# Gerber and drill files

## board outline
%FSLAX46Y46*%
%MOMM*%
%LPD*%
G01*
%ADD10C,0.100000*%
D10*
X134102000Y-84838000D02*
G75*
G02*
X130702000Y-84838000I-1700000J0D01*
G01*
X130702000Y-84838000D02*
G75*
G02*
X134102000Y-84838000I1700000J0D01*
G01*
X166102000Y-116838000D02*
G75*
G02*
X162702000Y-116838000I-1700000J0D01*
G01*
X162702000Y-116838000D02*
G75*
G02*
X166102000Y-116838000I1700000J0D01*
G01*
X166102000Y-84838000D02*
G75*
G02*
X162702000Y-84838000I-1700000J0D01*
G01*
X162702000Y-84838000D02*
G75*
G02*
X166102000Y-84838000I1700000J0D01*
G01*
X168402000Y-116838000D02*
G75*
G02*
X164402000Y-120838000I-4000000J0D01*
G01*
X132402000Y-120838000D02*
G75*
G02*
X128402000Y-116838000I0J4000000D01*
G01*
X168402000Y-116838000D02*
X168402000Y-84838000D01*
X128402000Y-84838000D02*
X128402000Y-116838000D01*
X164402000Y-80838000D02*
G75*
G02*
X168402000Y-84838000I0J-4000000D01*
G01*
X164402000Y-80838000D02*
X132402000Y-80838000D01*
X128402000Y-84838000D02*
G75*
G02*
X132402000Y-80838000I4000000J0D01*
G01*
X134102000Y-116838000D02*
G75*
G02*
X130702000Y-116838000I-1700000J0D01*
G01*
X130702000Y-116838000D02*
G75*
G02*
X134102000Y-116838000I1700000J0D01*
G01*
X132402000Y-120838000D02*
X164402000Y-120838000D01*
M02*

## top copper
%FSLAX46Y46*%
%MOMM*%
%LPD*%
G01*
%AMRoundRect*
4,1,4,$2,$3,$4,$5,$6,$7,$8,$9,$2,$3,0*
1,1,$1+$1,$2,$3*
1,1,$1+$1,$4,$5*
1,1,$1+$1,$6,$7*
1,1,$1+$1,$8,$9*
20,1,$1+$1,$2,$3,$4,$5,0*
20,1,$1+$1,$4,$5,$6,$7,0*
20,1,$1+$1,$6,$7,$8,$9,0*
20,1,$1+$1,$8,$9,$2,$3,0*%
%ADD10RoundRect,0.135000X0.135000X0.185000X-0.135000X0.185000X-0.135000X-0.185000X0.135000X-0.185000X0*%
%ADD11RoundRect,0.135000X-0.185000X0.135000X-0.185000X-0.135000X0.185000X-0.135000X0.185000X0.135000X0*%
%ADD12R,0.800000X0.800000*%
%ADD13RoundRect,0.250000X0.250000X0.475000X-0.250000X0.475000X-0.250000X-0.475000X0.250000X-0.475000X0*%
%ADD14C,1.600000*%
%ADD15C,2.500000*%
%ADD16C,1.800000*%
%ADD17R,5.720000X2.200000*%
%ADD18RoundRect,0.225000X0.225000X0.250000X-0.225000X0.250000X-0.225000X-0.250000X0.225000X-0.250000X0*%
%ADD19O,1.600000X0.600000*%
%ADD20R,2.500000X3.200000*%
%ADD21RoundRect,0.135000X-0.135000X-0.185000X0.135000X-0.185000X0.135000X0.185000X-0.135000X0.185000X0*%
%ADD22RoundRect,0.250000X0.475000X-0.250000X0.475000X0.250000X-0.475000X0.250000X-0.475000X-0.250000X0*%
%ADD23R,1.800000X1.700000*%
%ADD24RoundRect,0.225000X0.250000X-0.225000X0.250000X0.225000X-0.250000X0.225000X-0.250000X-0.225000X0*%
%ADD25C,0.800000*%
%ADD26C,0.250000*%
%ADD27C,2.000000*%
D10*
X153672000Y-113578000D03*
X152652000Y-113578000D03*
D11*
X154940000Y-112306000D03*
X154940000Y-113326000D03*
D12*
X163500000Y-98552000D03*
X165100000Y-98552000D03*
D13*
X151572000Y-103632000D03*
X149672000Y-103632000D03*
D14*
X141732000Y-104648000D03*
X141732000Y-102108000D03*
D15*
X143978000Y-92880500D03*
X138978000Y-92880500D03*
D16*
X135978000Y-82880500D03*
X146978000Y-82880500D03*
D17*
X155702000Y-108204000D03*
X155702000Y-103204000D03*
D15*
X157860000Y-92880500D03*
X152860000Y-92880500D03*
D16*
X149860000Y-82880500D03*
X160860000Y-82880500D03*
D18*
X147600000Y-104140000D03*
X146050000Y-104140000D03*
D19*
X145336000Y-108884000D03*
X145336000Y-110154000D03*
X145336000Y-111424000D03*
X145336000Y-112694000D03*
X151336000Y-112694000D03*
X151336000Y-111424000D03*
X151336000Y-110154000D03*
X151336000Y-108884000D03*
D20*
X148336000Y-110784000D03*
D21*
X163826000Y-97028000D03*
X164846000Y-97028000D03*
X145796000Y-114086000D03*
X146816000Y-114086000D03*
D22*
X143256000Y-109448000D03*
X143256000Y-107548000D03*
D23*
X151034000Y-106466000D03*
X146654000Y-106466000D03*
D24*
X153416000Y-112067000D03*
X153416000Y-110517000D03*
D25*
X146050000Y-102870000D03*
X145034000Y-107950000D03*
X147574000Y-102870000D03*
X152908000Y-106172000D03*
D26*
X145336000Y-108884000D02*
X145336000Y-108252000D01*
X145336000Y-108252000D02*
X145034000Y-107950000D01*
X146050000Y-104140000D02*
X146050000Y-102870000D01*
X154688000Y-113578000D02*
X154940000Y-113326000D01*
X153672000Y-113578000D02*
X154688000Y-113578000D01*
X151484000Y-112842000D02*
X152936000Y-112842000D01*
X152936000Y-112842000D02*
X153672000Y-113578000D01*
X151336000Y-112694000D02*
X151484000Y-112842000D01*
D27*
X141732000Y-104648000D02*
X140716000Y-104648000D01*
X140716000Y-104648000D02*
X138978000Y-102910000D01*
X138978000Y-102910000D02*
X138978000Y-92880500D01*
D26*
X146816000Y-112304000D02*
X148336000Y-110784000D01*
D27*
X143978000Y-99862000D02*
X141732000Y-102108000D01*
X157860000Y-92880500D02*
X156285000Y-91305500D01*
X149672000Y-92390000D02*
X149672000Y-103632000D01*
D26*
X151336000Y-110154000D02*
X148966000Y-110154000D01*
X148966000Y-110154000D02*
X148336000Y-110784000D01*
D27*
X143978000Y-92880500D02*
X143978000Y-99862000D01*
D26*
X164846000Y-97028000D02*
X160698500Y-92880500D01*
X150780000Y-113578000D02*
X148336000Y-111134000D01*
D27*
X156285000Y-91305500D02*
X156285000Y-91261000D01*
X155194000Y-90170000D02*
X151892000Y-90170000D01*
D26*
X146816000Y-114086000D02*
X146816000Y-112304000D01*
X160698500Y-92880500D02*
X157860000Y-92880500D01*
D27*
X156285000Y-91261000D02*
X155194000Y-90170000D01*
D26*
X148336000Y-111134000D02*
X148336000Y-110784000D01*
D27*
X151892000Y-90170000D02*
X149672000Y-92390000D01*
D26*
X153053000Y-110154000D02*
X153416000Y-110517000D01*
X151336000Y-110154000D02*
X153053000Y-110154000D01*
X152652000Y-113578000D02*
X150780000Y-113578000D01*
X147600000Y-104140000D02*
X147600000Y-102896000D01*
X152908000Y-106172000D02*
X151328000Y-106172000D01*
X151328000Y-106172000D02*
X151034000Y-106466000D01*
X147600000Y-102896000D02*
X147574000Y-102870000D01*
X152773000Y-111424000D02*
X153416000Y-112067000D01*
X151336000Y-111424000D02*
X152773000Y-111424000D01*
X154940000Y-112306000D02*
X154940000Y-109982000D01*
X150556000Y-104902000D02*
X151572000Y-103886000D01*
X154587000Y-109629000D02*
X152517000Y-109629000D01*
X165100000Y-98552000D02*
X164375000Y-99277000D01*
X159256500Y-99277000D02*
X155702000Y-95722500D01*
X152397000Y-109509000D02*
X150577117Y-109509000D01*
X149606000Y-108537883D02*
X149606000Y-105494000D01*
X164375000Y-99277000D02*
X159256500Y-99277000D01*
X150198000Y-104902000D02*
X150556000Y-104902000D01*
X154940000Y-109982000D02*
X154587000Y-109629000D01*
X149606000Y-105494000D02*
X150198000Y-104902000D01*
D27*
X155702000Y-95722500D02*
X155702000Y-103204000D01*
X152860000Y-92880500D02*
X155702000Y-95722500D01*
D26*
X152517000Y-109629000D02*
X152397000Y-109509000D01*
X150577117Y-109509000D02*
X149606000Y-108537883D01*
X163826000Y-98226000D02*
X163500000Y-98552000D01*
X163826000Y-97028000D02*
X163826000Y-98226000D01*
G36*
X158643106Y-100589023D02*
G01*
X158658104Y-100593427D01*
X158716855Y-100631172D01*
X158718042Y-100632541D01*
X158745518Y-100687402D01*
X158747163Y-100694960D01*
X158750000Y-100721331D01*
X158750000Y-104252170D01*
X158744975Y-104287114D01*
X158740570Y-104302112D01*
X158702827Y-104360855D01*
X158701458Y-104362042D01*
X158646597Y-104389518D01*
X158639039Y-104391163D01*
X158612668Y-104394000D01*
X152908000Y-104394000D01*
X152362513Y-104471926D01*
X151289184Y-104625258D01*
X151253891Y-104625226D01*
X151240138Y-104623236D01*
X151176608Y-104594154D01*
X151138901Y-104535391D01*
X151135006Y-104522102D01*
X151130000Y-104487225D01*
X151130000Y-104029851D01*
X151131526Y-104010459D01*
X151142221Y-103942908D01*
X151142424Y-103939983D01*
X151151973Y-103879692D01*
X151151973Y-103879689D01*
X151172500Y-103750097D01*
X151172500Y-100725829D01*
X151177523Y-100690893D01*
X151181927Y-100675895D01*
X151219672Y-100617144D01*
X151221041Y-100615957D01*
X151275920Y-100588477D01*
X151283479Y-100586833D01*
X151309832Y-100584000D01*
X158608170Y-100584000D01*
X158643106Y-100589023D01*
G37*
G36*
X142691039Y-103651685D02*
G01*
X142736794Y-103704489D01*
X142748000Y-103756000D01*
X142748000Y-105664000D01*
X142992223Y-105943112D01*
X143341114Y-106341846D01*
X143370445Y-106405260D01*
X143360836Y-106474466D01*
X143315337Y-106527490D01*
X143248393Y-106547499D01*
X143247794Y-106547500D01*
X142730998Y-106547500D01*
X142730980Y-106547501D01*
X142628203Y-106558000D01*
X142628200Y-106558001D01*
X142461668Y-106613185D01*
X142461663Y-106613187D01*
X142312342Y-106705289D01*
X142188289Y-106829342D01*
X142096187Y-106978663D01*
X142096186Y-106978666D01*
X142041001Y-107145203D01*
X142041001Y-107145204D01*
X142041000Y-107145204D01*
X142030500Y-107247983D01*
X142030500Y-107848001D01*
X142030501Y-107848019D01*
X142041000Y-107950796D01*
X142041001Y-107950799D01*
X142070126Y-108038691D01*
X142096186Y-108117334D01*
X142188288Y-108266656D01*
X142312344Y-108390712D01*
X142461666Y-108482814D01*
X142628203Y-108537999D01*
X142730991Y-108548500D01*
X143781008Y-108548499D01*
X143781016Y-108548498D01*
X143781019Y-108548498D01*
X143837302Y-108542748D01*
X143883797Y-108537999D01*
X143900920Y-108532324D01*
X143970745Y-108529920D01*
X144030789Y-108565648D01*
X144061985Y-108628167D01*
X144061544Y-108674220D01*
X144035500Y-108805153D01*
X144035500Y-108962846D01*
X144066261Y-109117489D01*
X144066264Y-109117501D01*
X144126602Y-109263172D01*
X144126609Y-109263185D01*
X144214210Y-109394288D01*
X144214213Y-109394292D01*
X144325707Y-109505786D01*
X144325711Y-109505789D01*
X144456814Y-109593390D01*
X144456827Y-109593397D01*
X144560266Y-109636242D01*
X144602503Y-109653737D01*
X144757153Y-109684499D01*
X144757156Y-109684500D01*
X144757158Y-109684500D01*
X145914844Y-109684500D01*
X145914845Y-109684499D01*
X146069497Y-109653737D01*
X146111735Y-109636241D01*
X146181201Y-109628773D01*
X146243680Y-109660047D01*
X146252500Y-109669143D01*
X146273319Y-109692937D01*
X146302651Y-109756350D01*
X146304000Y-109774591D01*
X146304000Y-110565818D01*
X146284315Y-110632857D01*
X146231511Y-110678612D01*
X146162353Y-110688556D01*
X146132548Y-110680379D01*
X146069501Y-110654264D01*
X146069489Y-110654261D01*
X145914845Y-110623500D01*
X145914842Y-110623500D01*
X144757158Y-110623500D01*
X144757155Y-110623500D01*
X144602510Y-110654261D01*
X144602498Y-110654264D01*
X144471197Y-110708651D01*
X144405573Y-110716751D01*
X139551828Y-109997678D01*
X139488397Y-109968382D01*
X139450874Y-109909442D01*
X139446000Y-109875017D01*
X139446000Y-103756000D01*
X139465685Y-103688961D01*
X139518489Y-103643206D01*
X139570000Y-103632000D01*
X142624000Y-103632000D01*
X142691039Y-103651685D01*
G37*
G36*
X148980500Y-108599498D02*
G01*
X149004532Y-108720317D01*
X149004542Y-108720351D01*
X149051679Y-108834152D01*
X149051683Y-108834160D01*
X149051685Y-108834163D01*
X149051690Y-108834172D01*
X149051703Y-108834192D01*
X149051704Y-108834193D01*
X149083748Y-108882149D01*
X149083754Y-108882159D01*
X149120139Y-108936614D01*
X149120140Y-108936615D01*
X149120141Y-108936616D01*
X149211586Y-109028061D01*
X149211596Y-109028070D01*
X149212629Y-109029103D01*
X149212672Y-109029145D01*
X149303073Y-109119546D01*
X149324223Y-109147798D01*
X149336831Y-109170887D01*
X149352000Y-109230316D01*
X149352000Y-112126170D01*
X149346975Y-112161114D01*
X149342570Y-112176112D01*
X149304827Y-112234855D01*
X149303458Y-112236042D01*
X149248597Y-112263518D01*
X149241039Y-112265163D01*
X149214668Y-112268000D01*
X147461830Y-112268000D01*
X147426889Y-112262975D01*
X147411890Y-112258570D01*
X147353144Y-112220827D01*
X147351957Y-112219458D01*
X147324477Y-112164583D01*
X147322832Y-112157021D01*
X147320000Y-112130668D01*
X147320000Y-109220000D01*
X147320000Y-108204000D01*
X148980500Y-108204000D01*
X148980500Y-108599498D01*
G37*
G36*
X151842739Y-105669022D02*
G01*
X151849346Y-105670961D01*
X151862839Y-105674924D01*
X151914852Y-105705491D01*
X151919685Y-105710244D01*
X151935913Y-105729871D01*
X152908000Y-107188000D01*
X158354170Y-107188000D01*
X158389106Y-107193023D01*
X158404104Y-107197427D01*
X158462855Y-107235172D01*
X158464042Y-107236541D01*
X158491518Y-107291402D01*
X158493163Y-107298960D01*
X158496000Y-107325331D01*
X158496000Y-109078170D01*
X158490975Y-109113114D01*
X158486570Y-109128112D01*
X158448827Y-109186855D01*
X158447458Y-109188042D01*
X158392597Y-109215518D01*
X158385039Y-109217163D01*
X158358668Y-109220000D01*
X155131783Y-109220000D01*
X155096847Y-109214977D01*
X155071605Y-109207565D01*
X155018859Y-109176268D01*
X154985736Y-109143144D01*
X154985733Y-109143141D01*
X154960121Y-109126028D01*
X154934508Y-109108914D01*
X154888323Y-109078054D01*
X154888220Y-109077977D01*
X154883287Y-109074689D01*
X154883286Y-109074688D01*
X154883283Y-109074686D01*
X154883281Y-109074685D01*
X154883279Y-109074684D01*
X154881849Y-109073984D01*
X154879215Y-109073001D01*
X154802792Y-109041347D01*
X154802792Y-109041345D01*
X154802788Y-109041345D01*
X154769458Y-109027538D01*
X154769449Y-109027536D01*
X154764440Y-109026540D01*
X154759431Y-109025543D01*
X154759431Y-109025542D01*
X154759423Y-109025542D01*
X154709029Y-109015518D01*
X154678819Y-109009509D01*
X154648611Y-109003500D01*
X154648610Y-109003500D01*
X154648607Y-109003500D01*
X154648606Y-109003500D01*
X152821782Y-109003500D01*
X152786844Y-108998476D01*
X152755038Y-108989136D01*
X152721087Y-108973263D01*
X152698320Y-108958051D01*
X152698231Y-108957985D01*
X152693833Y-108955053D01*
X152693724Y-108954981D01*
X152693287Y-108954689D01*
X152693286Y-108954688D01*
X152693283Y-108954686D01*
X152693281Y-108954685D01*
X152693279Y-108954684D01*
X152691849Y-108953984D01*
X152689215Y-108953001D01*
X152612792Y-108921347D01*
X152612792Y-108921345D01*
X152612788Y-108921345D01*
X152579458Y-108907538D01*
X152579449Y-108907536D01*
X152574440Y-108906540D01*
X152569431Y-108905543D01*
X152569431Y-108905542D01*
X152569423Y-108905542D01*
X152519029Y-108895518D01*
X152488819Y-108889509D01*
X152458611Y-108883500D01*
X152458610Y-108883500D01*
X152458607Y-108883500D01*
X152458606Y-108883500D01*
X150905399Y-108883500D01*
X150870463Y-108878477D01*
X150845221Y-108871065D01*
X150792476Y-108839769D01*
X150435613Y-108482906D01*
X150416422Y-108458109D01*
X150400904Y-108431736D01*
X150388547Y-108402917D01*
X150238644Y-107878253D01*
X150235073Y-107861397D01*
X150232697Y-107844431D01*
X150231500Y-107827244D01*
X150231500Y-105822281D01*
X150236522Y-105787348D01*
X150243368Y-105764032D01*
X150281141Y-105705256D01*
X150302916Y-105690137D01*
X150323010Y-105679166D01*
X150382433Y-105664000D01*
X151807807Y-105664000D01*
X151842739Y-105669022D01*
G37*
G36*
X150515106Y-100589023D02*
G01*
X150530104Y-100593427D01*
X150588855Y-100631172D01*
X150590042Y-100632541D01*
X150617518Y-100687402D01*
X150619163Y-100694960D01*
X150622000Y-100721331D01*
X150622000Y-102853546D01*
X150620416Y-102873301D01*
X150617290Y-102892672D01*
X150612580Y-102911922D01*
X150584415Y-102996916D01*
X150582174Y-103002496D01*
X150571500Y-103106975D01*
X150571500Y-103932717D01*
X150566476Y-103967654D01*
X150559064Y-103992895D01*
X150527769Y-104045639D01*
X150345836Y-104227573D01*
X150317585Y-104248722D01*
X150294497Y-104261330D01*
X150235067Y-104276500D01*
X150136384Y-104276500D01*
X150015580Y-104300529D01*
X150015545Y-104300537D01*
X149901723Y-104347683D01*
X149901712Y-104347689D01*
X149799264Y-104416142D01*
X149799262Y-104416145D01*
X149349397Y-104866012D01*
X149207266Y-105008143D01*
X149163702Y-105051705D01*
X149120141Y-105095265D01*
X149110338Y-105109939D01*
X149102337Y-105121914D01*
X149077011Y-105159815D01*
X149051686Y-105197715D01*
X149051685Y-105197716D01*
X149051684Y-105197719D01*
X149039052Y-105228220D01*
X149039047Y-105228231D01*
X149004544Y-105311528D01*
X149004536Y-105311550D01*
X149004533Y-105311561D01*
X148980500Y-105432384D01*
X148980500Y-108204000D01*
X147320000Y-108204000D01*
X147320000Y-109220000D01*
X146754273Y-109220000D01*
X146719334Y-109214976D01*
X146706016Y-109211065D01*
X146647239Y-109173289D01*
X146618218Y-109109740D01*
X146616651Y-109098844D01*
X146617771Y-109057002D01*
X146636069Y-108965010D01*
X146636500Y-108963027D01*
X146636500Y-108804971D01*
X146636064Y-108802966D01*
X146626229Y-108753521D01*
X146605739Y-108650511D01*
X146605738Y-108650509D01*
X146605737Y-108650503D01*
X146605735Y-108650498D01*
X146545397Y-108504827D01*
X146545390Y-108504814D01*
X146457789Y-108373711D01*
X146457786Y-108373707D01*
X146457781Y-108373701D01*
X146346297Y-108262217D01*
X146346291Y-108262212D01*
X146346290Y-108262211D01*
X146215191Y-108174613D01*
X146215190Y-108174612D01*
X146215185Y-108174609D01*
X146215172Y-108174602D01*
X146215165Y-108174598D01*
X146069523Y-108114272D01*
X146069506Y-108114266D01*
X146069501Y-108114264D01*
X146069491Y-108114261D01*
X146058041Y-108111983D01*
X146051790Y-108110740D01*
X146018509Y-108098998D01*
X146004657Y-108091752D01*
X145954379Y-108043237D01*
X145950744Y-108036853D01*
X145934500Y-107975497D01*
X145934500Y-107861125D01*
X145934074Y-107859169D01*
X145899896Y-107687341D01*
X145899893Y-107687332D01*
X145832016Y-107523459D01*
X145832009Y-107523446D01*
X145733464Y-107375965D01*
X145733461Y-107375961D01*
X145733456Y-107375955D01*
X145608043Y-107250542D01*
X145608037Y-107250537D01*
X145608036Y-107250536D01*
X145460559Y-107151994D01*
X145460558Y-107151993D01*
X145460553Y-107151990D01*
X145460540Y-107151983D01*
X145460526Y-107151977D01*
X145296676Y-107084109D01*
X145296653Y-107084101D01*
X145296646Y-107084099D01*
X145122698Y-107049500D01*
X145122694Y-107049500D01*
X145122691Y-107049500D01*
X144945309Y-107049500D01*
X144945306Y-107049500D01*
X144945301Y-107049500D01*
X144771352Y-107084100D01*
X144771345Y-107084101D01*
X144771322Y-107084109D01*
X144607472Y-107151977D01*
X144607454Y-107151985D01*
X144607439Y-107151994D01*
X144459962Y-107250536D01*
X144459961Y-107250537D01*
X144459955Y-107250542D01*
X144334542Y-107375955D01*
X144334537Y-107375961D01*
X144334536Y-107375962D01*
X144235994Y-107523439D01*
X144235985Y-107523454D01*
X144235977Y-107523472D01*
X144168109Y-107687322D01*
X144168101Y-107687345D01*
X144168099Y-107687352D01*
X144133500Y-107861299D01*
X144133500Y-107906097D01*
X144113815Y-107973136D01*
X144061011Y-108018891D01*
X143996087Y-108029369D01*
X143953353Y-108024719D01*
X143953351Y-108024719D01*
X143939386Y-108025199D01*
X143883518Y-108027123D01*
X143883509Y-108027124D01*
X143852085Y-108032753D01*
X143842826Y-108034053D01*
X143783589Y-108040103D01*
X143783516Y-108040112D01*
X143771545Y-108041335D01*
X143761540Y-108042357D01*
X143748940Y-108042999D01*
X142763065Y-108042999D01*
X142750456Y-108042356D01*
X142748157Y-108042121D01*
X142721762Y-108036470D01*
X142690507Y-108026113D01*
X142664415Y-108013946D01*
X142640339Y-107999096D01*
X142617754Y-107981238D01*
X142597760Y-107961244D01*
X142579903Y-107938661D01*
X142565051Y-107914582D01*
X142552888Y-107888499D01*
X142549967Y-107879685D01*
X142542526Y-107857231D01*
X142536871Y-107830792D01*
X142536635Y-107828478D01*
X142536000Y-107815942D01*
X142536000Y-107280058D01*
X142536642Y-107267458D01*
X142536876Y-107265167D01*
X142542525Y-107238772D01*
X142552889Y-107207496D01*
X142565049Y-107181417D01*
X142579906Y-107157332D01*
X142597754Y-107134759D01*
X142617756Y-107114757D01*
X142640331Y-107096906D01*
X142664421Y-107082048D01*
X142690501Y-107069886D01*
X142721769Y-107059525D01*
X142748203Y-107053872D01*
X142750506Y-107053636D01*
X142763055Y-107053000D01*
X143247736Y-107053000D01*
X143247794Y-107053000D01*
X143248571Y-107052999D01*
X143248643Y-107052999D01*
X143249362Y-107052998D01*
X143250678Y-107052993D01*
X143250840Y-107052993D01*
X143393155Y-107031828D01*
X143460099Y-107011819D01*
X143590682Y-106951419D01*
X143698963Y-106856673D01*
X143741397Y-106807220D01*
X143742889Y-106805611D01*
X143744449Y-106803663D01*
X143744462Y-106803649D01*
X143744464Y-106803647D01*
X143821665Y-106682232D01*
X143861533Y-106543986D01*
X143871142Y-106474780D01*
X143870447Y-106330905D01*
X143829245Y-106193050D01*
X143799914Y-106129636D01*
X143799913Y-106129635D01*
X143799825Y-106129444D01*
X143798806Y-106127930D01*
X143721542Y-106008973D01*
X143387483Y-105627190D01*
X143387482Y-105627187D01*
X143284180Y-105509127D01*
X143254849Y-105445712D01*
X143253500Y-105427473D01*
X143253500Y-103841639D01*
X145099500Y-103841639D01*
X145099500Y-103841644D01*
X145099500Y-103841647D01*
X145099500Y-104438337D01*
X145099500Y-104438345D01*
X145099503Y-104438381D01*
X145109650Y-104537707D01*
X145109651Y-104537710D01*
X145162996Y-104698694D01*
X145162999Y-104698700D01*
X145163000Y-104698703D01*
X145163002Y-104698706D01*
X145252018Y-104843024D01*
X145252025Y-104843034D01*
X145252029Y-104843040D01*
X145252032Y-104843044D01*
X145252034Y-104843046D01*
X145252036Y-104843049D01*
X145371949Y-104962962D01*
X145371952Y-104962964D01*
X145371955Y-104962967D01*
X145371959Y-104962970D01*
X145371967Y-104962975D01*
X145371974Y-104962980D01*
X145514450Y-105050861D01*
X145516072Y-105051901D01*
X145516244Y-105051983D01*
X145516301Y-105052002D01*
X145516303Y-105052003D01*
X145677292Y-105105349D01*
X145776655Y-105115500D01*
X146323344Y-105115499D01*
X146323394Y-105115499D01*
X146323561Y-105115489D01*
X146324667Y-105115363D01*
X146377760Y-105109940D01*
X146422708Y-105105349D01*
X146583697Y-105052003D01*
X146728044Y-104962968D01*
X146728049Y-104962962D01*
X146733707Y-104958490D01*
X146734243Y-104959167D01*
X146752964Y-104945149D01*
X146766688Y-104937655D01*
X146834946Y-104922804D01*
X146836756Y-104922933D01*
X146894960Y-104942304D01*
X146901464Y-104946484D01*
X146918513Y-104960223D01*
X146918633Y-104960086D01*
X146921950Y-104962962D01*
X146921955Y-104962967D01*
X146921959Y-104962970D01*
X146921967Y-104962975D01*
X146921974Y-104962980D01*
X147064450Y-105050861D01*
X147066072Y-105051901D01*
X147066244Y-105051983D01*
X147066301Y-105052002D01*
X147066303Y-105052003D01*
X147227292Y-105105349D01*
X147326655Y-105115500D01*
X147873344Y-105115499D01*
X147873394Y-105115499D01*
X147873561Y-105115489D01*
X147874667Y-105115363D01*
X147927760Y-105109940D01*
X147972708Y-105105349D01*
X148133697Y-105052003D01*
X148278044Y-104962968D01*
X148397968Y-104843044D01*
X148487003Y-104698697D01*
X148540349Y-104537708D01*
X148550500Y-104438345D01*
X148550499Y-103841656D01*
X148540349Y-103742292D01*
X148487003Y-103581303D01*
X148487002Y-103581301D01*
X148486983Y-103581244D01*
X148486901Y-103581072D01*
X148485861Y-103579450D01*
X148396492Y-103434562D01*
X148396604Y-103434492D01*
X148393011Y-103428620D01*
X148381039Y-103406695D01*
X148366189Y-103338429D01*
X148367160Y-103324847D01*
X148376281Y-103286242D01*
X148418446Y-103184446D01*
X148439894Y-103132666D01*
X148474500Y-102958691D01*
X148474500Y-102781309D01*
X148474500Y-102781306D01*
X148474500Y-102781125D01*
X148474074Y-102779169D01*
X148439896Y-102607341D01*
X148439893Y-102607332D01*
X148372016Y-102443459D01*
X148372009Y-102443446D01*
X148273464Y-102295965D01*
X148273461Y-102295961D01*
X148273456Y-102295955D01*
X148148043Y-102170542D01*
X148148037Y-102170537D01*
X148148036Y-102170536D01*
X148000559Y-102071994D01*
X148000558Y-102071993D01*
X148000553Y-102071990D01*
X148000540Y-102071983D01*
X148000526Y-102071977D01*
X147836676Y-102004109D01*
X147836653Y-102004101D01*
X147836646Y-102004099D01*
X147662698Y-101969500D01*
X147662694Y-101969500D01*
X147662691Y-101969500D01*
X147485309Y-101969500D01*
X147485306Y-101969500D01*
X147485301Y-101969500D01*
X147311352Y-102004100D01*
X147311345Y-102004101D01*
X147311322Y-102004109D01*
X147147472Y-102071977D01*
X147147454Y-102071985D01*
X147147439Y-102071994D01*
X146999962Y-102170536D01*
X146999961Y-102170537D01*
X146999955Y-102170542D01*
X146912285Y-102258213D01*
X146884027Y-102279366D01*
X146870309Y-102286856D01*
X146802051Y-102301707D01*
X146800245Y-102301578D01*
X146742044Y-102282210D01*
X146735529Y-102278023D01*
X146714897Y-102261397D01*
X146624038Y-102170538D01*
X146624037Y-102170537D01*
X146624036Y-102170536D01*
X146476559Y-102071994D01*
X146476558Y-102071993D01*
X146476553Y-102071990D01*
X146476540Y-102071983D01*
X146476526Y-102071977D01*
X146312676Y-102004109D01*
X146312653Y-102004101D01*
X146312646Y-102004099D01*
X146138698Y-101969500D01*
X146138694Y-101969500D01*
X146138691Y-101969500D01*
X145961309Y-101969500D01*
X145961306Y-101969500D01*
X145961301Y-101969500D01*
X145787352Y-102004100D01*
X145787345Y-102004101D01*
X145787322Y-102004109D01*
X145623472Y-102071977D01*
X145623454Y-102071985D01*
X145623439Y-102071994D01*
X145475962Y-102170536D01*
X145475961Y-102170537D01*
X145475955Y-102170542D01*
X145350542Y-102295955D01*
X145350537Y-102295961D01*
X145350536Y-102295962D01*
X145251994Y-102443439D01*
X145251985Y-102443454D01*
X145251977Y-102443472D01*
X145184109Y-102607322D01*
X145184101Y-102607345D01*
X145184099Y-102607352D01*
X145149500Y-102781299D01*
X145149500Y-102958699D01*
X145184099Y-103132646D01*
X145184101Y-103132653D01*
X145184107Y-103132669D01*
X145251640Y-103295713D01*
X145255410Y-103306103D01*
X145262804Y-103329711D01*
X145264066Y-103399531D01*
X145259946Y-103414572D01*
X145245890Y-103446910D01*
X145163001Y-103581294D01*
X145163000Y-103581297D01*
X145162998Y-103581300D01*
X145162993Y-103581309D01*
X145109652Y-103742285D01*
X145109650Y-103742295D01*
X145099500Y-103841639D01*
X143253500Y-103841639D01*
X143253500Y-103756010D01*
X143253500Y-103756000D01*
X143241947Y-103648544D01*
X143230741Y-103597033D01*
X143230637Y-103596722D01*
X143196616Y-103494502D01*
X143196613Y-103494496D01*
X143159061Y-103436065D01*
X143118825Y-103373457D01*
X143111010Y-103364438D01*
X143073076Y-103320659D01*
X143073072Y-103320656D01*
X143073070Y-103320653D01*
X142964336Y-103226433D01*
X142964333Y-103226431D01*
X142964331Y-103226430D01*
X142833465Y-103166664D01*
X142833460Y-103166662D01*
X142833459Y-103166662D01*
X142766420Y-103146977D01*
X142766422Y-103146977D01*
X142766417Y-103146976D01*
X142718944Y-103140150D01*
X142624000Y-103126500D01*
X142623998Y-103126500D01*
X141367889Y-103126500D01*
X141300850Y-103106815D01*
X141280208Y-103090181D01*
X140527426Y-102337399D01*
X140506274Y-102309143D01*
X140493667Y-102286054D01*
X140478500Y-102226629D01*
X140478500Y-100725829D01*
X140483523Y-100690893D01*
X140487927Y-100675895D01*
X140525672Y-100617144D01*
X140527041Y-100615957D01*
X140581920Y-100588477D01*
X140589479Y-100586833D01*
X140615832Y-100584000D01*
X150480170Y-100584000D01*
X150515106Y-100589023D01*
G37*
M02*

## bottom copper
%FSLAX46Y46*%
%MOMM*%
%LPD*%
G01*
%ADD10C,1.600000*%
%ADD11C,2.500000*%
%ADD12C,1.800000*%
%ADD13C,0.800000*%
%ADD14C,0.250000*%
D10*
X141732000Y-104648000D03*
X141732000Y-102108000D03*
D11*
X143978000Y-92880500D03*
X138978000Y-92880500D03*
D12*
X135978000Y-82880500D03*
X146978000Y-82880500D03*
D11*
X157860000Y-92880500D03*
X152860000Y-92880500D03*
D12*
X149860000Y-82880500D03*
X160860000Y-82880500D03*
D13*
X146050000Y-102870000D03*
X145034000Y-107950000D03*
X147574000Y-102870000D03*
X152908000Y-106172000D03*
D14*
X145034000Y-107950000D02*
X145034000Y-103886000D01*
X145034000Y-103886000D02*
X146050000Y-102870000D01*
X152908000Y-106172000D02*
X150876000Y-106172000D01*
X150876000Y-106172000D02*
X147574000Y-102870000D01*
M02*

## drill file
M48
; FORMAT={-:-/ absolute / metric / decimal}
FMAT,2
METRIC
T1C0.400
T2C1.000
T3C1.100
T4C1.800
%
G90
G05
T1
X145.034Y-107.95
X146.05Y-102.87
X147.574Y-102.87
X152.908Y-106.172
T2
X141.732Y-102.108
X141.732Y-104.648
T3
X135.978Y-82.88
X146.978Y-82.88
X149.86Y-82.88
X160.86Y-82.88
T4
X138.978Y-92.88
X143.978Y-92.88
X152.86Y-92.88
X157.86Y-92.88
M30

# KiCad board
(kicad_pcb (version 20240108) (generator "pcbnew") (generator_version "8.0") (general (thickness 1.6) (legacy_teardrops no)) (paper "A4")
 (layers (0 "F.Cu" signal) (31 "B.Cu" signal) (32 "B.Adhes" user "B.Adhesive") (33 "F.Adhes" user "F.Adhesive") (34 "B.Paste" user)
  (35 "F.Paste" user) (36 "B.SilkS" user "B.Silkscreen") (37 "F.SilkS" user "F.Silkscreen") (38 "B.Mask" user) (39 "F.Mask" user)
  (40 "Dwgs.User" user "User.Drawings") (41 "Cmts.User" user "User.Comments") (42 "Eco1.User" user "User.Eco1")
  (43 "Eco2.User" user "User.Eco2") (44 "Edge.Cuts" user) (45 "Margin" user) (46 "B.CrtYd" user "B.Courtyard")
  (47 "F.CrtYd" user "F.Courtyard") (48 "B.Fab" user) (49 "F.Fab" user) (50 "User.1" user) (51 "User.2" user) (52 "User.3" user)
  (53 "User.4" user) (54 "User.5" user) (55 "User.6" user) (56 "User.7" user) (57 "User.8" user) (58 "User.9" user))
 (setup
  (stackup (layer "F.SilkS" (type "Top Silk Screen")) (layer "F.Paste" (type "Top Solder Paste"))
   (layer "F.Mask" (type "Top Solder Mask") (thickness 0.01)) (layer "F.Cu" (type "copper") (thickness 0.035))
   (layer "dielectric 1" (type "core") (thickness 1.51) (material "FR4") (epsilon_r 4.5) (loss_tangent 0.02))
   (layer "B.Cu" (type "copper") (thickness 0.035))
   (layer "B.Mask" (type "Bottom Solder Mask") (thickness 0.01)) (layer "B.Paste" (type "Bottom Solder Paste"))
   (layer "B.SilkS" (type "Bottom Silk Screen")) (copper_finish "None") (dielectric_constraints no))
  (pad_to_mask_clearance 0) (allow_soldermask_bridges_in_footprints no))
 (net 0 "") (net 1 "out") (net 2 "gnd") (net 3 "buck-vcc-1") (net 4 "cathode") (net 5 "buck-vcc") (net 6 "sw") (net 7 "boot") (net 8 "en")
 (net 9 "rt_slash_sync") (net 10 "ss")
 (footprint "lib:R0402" (layer "F.Cu") (at 153.162 113.578 180)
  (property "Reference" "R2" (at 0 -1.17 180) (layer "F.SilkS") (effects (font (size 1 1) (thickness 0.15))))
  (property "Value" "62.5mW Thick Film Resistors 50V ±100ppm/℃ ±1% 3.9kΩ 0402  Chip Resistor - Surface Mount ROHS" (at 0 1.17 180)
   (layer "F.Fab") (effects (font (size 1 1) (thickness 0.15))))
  (pad "1" smd roundrect (at -0.51 0 180) (size 0.54 0.64) (layers "F.Cu" "F.Paste" "F.Mask") (roundrect_rratio 0.25) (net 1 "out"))
  (pad "2" smd roundrect (at 0.51 0 180) (size 0.54 0.64) (layers "F.Cu" "F.Paste" "F.Mask") (roundrect_rratio 0.25) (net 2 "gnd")))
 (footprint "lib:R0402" (layer "F.Cu") (at 154.94 112.816 -90)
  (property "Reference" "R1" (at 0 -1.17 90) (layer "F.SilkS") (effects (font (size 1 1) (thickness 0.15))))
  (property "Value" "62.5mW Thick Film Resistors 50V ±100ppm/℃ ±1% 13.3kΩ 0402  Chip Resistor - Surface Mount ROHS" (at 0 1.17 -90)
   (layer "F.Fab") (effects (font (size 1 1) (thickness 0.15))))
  (pad "1" smd roundrect (at -0.51 0 270) (size 0.54 0.64) (layers "F.Cu" "F.Paste" "F.Mask") (roundrect_rratio 0.25) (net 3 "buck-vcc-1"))
  (pad "2" smd roundrect (at 0.51 0 270) (size 0.54 0.64) (layers "F.Cu" "F.Paste" "F.Mask") (roundrect_rratio 0.25) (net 1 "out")))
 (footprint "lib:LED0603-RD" (layer "F.Cu") (at 164.3 98.552)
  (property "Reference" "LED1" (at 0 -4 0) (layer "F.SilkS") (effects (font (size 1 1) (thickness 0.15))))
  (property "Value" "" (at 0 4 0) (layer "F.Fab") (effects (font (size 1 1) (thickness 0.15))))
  (pad "1" smd rect (at -0.8 0 90) (size 0.8 0.8) (layers "F.Cu" "F.Paste" "F.Mask") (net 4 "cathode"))
  (pad "2" smd rect (at 0.8 0 90) (size 0.8 0.8) (layers "F.Cu" "F.Paste" "F.Mask") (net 3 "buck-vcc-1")))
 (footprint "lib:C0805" (layer "F.Cu") (at 150.622 103.632 180)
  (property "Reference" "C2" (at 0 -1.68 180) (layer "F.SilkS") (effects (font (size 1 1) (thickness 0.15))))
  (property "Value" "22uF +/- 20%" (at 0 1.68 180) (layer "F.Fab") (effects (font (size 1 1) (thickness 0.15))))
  (pad "1" smd roundrect (at -0.95 0 180) (size 1 1.45) (layers "F.Cu" "F.Paste" "F.Mask") (roundrect_rratio 0.25) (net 3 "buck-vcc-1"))
  (pad "2" smd roundrect (at 0.95 0 180) (size 1 1.45) (layers "F.Cu" "F.Paste" "F.Mask") (roundrect_rratio 0.25) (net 2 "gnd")))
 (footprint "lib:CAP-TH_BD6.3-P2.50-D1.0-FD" (layer "F.Cu") (at 141.732 103.378 90)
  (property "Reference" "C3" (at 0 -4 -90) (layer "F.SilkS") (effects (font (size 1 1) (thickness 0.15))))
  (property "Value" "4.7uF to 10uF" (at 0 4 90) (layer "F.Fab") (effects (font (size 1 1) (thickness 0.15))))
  (pad "1" thru_hole circle (at -1.27 0 90) (size 1.6 1.6) (drill 0.999998) (layers "*.Cu" "*.Mask") (remove_unused_layers no)
   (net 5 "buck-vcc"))
  (pad "2" thru_hole circle (at 1.27 0 90) (size 1.6 1.6) (drill 0.999998) (layers "*.Cu" "*.Mask") (remove_unused_layers no) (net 2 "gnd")))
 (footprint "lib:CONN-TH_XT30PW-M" (layer "F.Cu") (at 141.478 87.8805 180)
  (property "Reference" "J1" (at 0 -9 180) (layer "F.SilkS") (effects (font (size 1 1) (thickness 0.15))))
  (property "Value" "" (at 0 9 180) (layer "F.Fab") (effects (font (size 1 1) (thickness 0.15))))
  (pad "1" thru_hole circle (at -2.5 -5 180) (size 2.5 2.5) (drill 1.799996) (layers "*.Cu" "*.Mask") (remove_unused_layers no)
   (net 2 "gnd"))
  (pad "2" thru_hole circle (at 2.5 -5 180) (size 2.5 2.5) (drill 1.799996) (layers "*.Cu" "*.Mask") (remove_unused_layers no)
   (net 5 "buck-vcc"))
  (pad "3" thru_hole circle (at 5.5 5 180) (size 1.8 1.8) (drill 1.100023) (layers "*.Cu" "*.Mask") (remove_unused_layers no))
  (pad "4" thru_hole circle (at -5.5 5 180) (size 1.8 1.8) (drill 1.100023) (layers "*.Cu" "*.Mask") (remove_unused_layers no)))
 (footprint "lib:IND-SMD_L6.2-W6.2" (layer "F.Cu") (at 155.702 105.704 90)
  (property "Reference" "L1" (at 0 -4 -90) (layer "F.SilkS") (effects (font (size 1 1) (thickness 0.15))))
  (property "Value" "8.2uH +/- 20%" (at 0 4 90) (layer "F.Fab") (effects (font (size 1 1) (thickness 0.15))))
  (pad "1" smd rect (at -2.5 0 90) (size 2.2 5.72) (layers "F.Cu" "F.Paste" "F.Mask") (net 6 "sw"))
  (pad "2" smd rect (at 2.5 0 90) (size 2.2 5.72) (layers "F.Cu" "F.Paste" "F.Mask") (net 3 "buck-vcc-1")))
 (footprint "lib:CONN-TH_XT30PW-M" (layer "F.Cu") (at 155.36 87.8805 180)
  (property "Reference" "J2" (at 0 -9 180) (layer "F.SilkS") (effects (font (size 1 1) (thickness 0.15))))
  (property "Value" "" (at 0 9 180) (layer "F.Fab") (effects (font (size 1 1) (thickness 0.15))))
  (pad "1" thru_hole circle (at -2.5 -5 180) (size 2.5 2.5) (drill 1.799996) (layers "*.Cu" "*.Mask") (remove_unused_layers no)
   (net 2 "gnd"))
  (pad "2" thru_hole circle (at 2.5 -5 180) (size 2.5 2.5) (drill 1.799996) (layers "*.Cu" "*.Mask") (remove_unused_layers no)
   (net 3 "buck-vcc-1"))
  (pad "3" thru_hole circle (at 5.5 5 180) (size 1.8 1.8) (drill 1.100023) (layers "*.Cu" "*.Mask") (remove_unused_layers no))
  (pad "4" thru_hole circle (at -5.5 5 180) (size 1.8 1.8) (drill 1.100023) (layers "*.Cu" "*.Mask") (remove_unused_layers no)))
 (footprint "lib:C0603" (layer "F.Cu") (at 146.825 104.14 180)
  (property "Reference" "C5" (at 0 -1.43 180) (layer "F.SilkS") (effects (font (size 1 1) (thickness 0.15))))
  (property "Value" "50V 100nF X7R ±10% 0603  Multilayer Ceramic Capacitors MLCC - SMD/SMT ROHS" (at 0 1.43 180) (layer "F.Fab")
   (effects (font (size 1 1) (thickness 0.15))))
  (pad "1" smd roundrect (at -0.775 0 180) (size 0.9 0.95) (layers "F.Cu" "F.Paste" "F.Mask") (roundrect_rratio 0.25) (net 6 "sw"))
  (pad "2" smd roundrect (at 0.775 0 180) (size 0.9 0.95) (layers "F.Cu" "F.Paste" "F.Mask") (roundrect_rratio 0.25) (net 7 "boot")))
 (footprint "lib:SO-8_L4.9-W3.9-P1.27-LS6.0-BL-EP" (layer "F.Cu") (at 148.336 110.784 -90)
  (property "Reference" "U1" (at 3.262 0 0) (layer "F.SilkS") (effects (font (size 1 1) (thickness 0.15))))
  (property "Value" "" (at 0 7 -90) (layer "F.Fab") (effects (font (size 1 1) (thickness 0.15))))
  (pad "1" smd oval (at -1.9 3 270) (size 0.6 1.6) (layers "F.Cu" "F.Paste" "F.Mask") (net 7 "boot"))
  (pad "2" smd oval (at -0.63 3 270) (size 0.6 1.6) (layers "F.Cu" "F.Paste" "F.Mask") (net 5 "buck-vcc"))
  (pad "3" smd oval (at 0.64 3 270) (size 0.6 1.6) (layers "F.Cu" "F.Paste" "F.Mask") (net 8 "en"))
  (pad "4" smd oval (at 1.91 3 270) (size 0.6 1.6) (layers "F.Cu" "F.Paste" "F.Mask") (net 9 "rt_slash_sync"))
  (pad "5" smd oval (at 1.91 -3 270) (size 0.6 1.6) (layers "F.Cu" "F.Paste" "F.Mask") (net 1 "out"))
  (pad "6" smd oval (at 0.64 -3 270) (size 0.6 1.6) (layers "F.Cu" "F.Paste" "F.Mask") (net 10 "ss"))
  (pad "7" smd oval (at -0.63 -3 270) (size 0.6 1.6) (layers "F.Cu" "F.Paste" "F.Mask") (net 2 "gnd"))
  (pad "8" smd oval (at -1.9 -3 270) (size 0.6 1.6) (layers "F.Cu" "F.Paste" "F.Mask") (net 6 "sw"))
  (pad "9" smd rect (at 0 0 270) (size 3.2 2.5) (layers "F.Cu" "F.Paste" "F.Mask") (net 2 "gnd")))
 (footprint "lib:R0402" (layer "F.Cu") (at 164.336 97.028)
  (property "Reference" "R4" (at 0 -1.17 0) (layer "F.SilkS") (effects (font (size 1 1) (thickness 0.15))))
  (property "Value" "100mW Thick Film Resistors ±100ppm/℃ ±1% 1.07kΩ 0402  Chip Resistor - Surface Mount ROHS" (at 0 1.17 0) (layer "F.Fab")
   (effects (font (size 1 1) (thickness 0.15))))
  (pad "1" smd roundrect (at -0.51 0) (size 0.54 0.64) (layers "F.Cu" "F.Paste" "F.Mask") (roundrect_rratio 0.25) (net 4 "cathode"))
  (pad "2" smd roundrect (at 0.51 0) (size 0.54 0.64) (layers "F.Cu" "F.Paste" "F.Mask") (roundrect_rratio 0.25) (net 2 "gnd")))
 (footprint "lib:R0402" (layer "F.Cu") (at 146.306 114.086)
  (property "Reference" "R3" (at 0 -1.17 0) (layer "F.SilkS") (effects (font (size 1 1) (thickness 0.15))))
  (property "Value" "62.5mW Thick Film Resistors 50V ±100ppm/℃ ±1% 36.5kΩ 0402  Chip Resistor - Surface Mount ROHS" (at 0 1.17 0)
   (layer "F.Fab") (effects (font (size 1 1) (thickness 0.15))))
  (pad "1" smd roundrect (at -0.51 0) (size 0.54 0.64) (layers "F.Cu" "F.Paste" "F.Mask") (roundrect_rratio 0.25) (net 9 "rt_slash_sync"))
  (pad "2" smd roundrect (at 0.51 0) (size 0.54 0.64) (layers "F.Cu" "F.Paste" "F.Mask") (roundrect_rratio 0.25) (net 2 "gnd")))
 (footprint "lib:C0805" (layer "F.Cu") (at 143.256 108.498 90)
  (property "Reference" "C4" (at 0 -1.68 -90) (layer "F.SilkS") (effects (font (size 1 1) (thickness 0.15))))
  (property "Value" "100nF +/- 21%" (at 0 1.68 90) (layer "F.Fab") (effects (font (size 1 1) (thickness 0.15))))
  (pad "1" smd roundrect (at -0.95 0 90) (size 1 1.45) (layers "F.Cu" "F.Paste" "F.Mask") (roundrect_rratio 0.25) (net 5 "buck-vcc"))
  (pad "2" smd roundrect (at 0.95 0 90) (size 1 1.45) (layers "F.Cu" "F.Paste" "F.Mask") (roundrect_rratio 0.25) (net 2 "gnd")))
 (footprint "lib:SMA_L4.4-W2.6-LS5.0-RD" (layer "F.Cu") (at 148.844 106.466 180)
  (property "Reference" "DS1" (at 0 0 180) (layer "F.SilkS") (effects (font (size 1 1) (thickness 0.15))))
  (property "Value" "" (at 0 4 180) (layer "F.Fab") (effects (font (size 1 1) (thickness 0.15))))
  (pad "1" smd rect (at -2.19 0 180) (size 1.8 1.7) (layers "F.Cu" "F.Paste" "F.Mask") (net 6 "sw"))
  (pad "2" smd rect (at 2.19 0 180) (size 1.8 1.7) (layers "F.Cu" "F.Paste" "F.Mask") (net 2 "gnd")))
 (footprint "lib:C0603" (layer "F.Cu") (at 153.416 111.292 90)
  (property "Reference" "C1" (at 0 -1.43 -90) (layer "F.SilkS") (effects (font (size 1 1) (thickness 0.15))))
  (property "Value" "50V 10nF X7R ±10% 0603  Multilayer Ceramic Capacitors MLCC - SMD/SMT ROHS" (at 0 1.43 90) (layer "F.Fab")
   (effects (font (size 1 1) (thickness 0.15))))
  (pad "1" smd roundrect (at -0.775 0 90) (size 0.9 0.95) (layers "F.Cu" "F.Paste" "F.Mask") (roundrect_rratio 0.25) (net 10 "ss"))
  (pad "2" smd roundrect (at 0.775 0 90) (size 0.9 0.95) (layers "F.Cu" "F.Paste" "F.Mask") (roundrect_rratio 0.25) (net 2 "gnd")))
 (gr_circle (center 132.402 84.838) (end 134.102 84.838) (stroke (width 0.1) (type solid)) (fill none) (layer "Edge.Cuts"))
 (gr_circle (center 164.402 116.838) (end 166.102 116.838) (stroke (width 0.1) (type solid)) (fill none) (layer "Edge.Cuts"))
 (gr_circle (center 164.402 84.838) (end 166.102 84.838) (stroke (width 0.1) (type solid)) (fill none) (layer "Edge.Cuts"))
 (gr_arc (start 168.402 116.838) (mid 167.230427 119.666427) (end 164.402 120.838) (stroke (width 0.1) (type solid)) (layer "Edge.Cuts"))
 (gr_arc (start 132.402 120.838) (mid 129.573573 119.666427) (end 128.402 116.838) (stroke (width 0.1) (type solid)) (layer "Edge.Cuts"))
 (gr_line (start 168.402 116.838) (end 168.402 84.838) (stroke (width 0.1) (type solid)) (layer "Edge.Cuts"))
 (gr_line (start 128.402 84.838) (end 128.402 116.838) (stroke (width 0.1) (type solid)) (layer "Edge.Cuts"))
 (gr_arc (start 164.402 80.838) (mid 167.230427 82.009573) (end 168.402 84.838) (stroke (width 0.1) (type solid)) (layer "Edge.Cuts"))
 (gr_line (start 164.402 80.838) (end 132.402 80.838) (stroke (width 0.1) (type solid)) (layer "Edge.Cuts"))
 (gr_arc (start 128.402 84.838) (mid 129.573573 82.009573) (end 132.402 80.838) (stroke (width 0.1) (type solid)) (layer "Edge.Cuts"))
 (gr_circle (center 132.402 116.838) (end 134.102 116.838) (stroke (width 0.1) (type solid)) (fill none) (layer "Edge.Cuts"))
 (gr_line (start 132.402 120.838) (end 164.402 120.838) (stroke (width 0.1) (type solid)) (layer "Edge.Cuts"))
 (segment (start 145.336 108.884) (end 145.336 108.252) (width 0.25) (layer "F.Cu") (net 7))
 (segment (start 145.336 108.252) (end 145.034 107.95) (width 0.25) (layer "F.Cu") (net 7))
 (segment (start 146.05 104.14) (end 146.05 102.87) (width 0.25) (layer "F.Cu") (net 7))
 (via (at 146.05 102.87) (size 0.8) (drill 0.4) (layers "F.Cu" "B.Cu") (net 7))
 (via (at 145.034 107.95) (size 0.8) (drill 0.4) (layers "F.Cu" "B.Cu") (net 7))
 (segment (start 145.034 107.95) (end 145.034 103.886) (width 0.25) (layer "B.Cu") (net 7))
 (segment (start 145.034 103.886) (end 146.05 102.87) (width 0.25) (layer "B.Cu") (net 7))
 (segment (start 154.688 113.578) (end 154.94 113.326) (width 0.25) (layer "F.Cu") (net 1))
 (segment (start 153.672 113.578) (end 154.688 113.578) (width 0.25) (layer "F.Cu") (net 1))
 (segment (start 151.484 112.842) (end 152.936 112.842) (width 0.25) (layer "F.Cu") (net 1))
 (segment (start 152.936 112.842) (end 153.672 113.578) (width 0.25) (layer "F.Cu") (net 1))
 (segment (start 151.336 112.694) (end 151.484 112.842) (width 0.25) (layer "F.Cu") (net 1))
 (segment (start 141.732 104.648) (end 140.716 104.648) (width 2) (layer "F.Cu") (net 5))
 (segment (start 140.716 104.648) (end 138.978 102.91) (width 2) (layer "F.Cu") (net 5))
 (segment (start 138.978 102.91) (end 138.978 92.8805) (width 2) (layer "F.Cu") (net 5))
 (segment (start 146.816 112.304) (end 148.336 110.784) (width 0.25) (layer "F.Cu") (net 2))
 (segment (start 143.978 99.862) (end 141.732 102.108) (width 2) (layer "F.Cu") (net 2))
 (segment (start 157.86 92.8805) (end 156.285 91.3055) (width 2) (layer "F.Cu") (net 2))
 (segment (start 149.672 92.39) (end 149.672 103.632) (width 2) (layer "F.Cu") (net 2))
 (segment (start 151.336 110.154) (end 148.966 110.154) (width 0.25) (layer "F.Cu") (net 2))
 (segment (start 148.966 110.154) (end 148.336 110.784) (width 0.25) (layer "F.Cu") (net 2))
 (segment (start 143.978 92.8805) (end 143.978 99.862) (width 2) (layer "F.Cu") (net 2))
 (segment (start 164.846 97.028) (end 160.6985 92.8805) (width 0.25) (layer "F.Cu") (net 2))
 (segment (start 150.78 113.578) (end 148.336 111.134) (width 0.25) (layer "F.Cu") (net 2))
 (segment (start 156.285 91.3055) (end 156.285 91.261) (width 2) (layer "F.Cu") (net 2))
 (segment (start 155.194 90.17) (end 151.892 90.17) (width 2) (layer "F.Cu") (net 2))
 (segment (start 146.816 114.086) (end 146.816 112.304) (width 0.25) (layer "F.Cu") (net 2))
 (segment (start 160.6985 92.8805) (end 157.86 92.8805) (width 0.25) (layer "F.Cu") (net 2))
 (segment (start 156.285 91.261) (end 155.194 90.17) (width 2) (layer "F.Cu") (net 2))
 (segment (start 148.336 111.134) (end 148.336 110.784) (width 0.25) (layer "F.Cu") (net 2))
 (segment (start 151.892 90.17) (end 149.672 92.39) (width 2) (layer "F.Cu") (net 2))
 (segment (start 153.053 110.154) (end 153.416 110.517) (width 0.25) (layer "F.Cu") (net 2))
 (segment (start 151.336 110.154) (end 153.053 110.154) (width 0.25) (layer "F.Cu") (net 2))
 (segment (start 152.652 113.578) (end 150.78 113.578) (width 0.25) (layer "F.Cu") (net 2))
 (segment (start 147.6 104.14) (end 147.6 102.896) (width 0.25) (layer "F.Cu") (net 6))
 (segment (start 152.908 106.172) (end 151.328 106.172) (width 0.25) (layer "F.Cu") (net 6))
 (segment (start 151.328 106.172) (end 151.034 106.466) (width 0.25) (layer "F.Cu") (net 6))
 (segment (start 147.6 102.896) (end 147.574 102.87) (width 0.25) (layer "F.Cu") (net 6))
 (via (at 147.574 102.87) (size 0.8) (drill 0.4) (layers "F.Cu" "B.Cu") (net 6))
 (via (at 152.908 106.172) (size 0.8) (drill 0.4) (layers "F.Cu" "B.Cu") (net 6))
 (segment (start 152.908 106.172) (end 150.876 106.172) (width 0.25) (layer "B.Cu") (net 6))
 (segment (start 150.876 106.172) (end 147.574 102.87) (width 0.25) (layer "B.Cu") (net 6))
 (segment (start 152.773 111.424) (end 153.416 112.067) (width 0.25) (layer "F.Cu") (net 10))
 (segment (start 151.336 111.424) (end 152.773 111.424) (width 0.25) (layer "F.Cu") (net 10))
 (segment (start 154.94 112.306) (end 154.94 109.982) (width 0.25) (layer "F.Cu") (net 3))
 (segment (start 150.556 104.902) (end 151.572 103.886) (width 0.25) (layer "F.Cu") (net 3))
 (segment (start 154.587 109.629) (end 152.517 109.629) (width 0.25) (layer "F.Cu") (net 3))
 (segment (start 165.1 98.552) (end 164.375 99.277) (width 0.25) (layer "F.Cu") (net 3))
 (segment (start 159.2565 99.277) (end 155.702 95.7225) (width 0.25) (layer "F.Cu") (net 3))
 (segment (start 152.397 109.509) (end 150.577117 109.509) (width 0.25) (layer "F.Cu") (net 3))
 (segment (start 149.606 108.537883) (end 149.606 105.494) (width 0.25) (layer "F.Cu") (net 3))
 (segment (start 164.375 99.277) (end 159.2565 99.277) (width 0.25) (layer "F.Cu") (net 3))
 (segment (start 150.198 104.902) (end 150.556 104.902) (width 0.25) (layer "F.Cu") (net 3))
 (segment (start 154.94 109.982) (end 154.587 109.629) (width 0.25) (layer "F.Cu") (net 3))
 (segment (start 149.606 105.494) (end 150.198 104.902) (width 0.25) (layer "F.Cu") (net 3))
 (segment (start 155.702 95.7225) (end 155.702 103.204) (width 2) (layer "F.Cu") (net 3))
 (segment (start 152.86 92.8805) (end 155.702 95.7225) (width 2) (layer "F.Cu") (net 3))
 (segment (start 152.517 109.629) (end 152.397 109.509) (width 0.25) (layer "F.Cu") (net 3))
 (segment (start 150.577117 109.509) (end 149.606 108.537883) (width 0.25) (layer "F.Cu") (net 3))
 (segment (start 163.826 98.226) (end 163.5 98.552) (width 0.25) (layer "F.Cu") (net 4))
 (segment (start 163.826 97.028) (end 163.826 98.226) (width 0.25) (layer "F.Cu") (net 4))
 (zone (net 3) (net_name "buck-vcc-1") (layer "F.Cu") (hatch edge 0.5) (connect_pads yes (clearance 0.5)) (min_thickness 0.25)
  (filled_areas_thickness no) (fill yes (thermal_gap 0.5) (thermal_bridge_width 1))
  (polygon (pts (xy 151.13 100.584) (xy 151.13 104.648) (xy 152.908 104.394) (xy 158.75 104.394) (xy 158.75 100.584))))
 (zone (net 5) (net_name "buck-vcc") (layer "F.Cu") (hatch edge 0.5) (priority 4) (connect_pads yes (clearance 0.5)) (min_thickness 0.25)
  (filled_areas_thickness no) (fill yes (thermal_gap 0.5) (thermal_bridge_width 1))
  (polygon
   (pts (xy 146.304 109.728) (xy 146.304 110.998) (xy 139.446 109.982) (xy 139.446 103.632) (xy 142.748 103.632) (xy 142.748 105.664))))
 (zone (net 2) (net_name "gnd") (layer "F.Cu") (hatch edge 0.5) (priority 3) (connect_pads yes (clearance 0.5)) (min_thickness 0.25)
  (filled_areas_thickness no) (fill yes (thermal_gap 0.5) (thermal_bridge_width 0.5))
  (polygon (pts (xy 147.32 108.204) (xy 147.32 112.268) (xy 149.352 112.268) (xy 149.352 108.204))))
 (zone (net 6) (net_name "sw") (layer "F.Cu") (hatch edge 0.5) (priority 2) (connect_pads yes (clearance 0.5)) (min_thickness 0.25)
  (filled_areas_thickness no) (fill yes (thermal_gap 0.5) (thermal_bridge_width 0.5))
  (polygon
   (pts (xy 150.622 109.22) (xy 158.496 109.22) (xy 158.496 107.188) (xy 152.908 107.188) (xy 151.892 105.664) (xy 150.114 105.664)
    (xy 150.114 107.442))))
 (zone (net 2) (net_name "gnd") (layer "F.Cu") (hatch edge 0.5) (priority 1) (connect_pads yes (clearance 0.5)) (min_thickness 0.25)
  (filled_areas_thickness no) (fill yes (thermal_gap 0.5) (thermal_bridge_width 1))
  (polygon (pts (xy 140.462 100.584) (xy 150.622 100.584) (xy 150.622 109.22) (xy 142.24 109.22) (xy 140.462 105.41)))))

